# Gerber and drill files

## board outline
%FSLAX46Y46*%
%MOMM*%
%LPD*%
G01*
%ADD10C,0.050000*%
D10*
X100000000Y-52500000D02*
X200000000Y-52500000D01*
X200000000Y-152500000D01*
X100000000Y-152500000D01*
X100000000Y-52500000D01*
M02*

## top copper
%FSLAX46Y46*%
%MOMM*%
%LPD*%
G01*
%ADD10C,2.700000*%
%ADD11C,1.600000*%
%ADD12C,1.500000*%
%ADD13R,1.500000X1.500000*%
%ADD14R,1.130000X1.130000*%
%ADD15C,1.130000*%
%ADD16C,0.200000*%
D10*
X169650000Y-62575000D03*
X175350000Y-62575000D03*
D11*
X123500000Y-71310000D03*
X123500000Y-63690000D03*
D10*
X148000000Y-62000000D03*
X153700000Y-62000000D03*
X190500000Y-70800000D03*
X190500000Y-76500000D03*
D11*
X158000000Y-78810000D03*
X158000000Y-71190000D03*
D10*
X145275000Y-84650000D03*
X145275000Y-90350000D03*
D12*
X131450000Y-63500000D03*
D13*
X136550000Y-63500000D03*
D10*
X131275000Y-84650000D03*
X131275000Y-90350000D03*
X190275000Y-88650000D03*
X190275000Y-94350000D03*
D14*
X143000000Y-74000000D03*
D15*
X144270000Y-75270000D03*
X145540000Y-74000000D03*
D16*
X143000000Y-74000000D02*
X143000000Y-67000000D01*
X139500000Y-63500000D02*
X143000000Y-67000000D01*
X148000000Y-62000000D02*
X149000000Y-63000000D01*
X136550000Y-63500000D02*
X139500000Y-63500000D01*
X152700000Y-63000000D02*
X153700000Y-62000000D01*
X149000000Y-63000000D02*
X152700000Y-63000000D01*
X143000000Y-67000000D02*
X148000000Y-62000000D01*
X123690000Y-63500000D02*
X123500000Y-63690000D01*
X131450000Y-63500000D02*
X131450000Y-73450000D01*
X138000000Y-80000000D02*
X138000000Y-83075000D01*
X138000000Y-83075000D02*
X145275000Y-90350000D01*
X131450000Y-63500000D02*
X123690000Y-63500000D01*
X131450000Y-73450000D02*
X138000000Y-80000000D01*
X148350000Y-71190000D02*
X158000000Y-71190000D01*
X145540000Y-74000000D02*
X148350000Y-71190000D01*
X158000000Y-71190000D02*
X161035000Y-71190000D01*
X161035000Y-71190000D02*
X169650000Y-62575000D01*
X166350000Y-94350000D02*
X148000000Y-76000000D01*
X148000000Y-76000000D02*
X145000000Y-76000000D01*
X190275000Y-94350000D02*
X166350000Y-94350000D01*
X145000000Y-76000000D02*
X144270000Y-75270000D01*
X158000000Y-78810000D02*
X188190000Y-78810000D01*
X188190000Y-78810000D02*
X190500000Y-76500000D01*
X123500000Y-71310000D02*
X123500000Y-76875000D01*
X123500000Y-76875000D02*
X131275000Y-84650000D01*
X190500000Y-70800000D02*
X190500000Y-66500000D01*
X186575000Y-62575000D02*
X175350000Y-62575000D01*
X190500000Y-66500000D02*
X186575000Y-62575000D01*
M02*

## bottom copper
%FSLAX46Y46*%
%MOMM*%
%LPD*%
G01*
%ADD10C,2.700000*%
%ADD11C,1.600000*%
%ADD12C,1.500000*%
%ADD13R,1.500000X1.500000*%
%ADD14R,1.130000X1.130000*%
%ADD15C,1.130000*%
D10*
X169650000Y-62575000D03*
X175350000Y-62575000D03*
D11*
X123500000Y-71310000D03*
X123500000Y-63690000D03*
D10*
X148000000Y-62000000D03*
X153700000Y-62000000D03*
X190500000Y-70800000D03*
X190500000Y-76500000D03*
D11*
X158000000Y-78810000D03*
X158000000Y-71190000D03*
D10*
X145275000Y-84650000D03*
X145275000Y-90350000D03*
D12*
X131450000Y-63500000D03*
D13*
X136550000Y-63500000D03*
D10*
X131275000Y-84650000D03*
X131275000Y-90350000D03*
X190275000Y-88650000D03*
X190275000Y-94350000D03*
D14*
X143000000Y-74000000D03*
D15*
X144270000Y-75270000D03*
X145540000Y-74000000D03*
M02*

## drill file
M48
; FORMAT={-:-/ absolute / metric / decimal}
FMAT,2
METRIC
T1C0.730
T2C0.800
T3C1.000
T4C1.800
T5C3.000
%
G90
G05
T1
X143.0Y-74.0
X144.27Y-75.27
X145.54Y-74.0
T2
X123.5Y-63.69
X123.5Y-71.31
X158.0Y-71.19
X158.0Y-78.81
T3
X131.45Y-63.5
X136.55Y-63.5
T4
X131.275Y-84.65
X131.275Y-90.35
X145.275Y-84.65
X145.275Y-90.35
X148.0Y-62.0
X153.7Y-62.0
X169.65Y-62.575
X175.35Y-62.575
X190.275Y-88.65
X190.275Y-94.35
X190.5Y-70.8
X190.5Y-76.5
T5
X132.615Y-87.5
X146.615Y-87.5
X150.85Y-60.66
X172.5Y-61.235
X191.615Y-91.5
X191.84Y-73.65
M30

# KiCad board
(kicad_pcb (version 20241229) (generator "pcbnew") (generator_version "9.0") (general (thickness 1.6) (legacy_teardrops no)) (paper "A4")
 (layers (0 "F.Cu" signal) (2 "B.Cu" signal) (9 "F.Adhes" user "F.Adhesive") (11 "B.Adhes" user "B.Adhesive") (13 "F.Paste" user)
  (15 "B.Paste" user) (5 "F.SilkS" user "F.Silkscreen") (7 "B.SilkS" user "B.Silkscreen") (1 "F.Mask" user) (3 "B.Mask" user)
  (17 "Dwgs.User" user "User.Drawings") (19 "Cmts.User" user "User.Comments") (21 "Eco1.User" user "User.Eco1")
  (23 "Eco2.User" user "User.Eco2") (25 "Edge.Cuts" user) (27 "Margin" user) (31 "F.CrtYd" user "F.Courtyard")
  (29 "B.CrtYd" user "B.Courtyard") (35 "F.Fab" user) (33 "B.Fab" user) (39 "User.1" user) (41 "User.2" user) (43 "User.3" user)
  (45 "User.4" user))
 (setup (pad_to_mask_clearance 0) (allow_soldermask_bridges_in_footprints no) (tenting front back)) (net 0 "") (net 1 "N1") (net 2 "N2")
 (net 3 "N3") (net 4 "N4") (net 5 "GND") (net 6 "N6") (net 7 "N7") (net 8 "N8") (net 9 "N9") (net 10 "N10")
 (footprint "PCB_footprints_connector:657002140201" (layer "F.Cu") (at 172.5 62.575 180)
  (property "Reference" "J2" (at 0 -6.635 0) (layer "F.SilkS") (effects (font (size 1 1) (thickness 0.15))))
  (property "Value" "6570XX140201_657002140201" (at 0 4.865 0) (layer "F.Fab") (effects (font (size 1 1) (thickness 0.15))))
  (pad "" np_thru_hole circle (at 0 1.34 180) (size 3 3) (drill 3) (layers "*.Cu" "*.Mask"))
  (pad "1" thru_hole circle (at 2.85 0 180) (size 2.7 2.7) (drill 1.8) (layers "*.Cu" "*.Mask") (remove_unused_layers no) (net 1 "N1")
   (solder_mask_margin 0.102))
  (pad "2" thru_hole circle (at -2.85 0 180) (size 2.7 2.7) (drill 1.8) (layers "*.Cu" "*.Mask") (remove_unused_layers no) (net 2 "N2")
   (solder_mask_margin 0.102)))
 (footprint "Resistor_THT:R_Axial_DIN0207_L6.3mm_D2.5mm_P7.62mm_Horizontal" (layer "F.Cu") (at 123.5 71.31 90)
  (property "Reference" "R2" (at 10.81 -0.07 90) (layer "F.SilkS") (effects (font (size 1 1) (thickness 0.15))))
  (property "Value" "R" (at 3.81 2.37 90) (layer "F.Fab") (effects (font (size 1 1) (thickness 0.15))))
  (pad "1" thru_hole circle (at 0 0 90) (size 1.6 1.6) (drill 0.8) (layers "*.Cu" "*.Mask") (remove_unused_layers no) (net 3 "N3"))
  (pad "2" thru_hole circle (at 7.62 0 90) (size 1.6 1.6) (drill 0.8) (layers "*.Cu" "*.Mask") (remove_unused_layers no) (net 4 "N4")))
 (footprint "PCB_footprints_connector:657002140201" (layer "F.Cu") (at 150.85 62 180)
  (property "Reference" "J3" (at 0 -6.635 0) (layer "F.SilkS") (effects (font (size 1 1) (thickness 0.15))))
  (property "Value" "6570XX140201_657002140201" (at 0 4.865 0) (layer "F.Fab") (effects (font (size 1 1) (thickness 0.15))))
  (pad "" np_thru_hole circle (at 0 1.34 180) (size 3 3) (drill 3) (layers "*.Cu" "*.Mask"))
  (pad "1" thru_hole circle (at 2.85 0 180) (size 2.7 2.7) (drill 1.8) (layers "*.Cu" "*.Mask") (remove_unused_layers no) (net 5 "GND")
   (solder_mask_margin 0.102))
  (pad "2" thru_hole circle (at -2.85 0 180) (size 2.7 2.7) (drill 1.8) (layers "*.Cu" "*.Mask") (remove_unused_layers no) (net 5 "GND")
   (solder_mask_margin 0.102)))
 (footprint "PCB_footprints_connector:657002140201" (layer "F.Cu") (at 190.5 73.65 90)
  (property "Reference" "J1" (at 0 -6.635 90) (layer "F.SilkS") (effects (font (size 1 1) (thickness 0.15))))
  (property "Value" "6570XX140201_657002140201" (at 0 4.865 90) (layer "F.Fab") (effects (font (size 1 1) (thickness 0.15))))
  (pad "" np_thru_hole circle (at 0 1.34 90) (size 3 3) (drill 3) (layers "*.Cu" "*.Mask"))
  (pad "1" thru_hole circle (at 2.85 0 90) (size 2.7 2.7) (drill 1.8) (layers "*.Cu" "*.Mask") (remove_unused_layers no) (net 2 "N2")
   (solder_mask_margin 0.102))
  (pad "2" thru_hole circle (at -2.85 0 90) (size 2.7 2.7) (drill 1.8) (layers "*.Cu" "*.Mask") (remove_unused_layers no) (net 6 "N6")
   (solder_mask_margin 0.102)))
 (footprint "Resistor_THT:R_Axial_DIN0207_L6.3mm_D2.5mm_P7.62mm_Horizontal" (layer "F.Cu") (at 158 78.81 90)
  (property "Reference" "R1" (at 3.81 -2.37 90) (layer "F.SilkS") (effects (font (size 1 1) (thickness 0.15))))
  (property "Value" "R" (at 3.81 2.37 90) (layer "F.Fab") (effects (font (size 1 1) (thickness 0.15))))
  (pad "1" thru_hole circle (at 0 0 90) (size 1.6 1.6) (drill 0.8) (layers "*.Cu" "*.Mask") (remove_unused_layers no) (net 6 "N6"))
  (pad "2" thru_hole circle (at 7.62 0 90) (size 1.6 1.6) (drill 0.8) (layers "*.Cu" "*.Mask") (remove_unused_layers no) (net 1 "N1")))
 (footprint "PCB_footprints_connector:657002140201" (layer "F.Cu") (at 145.275 87.5 90)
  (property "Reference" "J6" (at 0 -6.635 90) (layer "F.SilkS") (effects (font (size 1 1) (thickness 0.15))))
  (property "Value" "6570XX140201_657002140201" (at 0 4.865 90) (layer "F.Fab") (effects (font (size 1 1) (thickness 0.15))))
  (pad "" np_thru_hole circle (at 0 1.34 90) (size 3 3) (drill 3) (layers "*.Cu" "*.Mask"))
  (pad "1" thru_hole circle (at 2.85 0 90) (size 2.7 2.7) (drill 1.8) (layers "*.Cu" "*.Mask") (remove_unused_layers no) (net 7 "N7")
   (solder_mask_margin 0.102))
  (pad "2" thru_hole circle (at -2.85 0 90) (size 2.7 2.7) (drill 1.8) (layers "*.Cu" "*.Mask") (remove_unused_layers no) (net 4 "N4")
   (solder_mask_margin 0.102)))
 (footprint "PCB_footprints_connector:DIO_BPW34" (layer "F.Cu") (at 134 63.5 180)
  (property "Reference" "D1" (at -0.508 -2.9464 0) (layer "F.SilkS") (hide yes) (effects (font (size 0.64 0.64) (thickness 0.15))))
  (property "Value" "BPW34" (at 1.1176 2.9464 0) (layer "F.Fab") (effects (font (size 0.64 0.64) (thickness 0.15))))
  (pad "A" thru_hole circle (at 2.55 0 180) (size 1.5 1.5) (drill 1) (layers "*.Cu" "*.Mask") (remove_unused_layers no) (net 4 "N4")
   (solder_mask_margin 0.102))
  (pad "C" thru_hole rect (at -2.55 0 180) (size 1.5 1.5) (drill 1) (layers "*.Cu" "*.Mask") (remove_unused_layers no) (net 5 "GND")
   (solder_mask_margin 0.102)))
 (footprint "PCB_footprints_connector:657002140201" (layer "F.Cu") (at 131.275 87.5 90)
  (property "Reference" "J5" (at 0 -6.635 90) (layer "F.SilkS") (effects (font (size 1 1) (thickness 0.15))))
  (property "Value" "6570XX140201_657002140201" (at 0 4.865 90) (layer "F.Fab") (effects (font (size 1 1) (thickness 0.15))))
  (pad "" np_thru_hole circle (at 0 1.34 90) (size 3 3) (drill 3) (layers "*.Cu" "*.Mask"))
  (pad "1" thru_hole circle (at 2.85 0 90) (size 2.7 2.7) (drill 1.8) (layers "*.Cu" "*.Mask") (remove_unused_layers no) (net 3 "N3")
   (solder_mask_margin 0.102))
  (pad "2" thru_hole circle (at -2.85 0 90) (size 2.7 2.7) (drill 1.8) (layers "*.Cu" "*.Mask") (remove_unused_layers no) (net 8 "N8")
   (solder_mask_margin 0.102)))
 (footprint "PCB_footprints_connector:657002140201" (layer "F.Cu") (at 190.275 91.5 90)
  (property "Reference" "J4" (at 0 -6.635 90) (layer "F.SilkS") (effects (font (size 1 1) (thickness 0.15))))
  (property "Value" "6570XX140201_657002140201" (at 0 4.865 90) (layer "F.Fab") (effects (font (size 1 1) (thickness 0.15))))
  (pad "" np_thru_hole circle (at 0 1.34 90) (size 3 3) (drill 3) (layers "*.Cu" "*.Mask"))
  (pad "1" thru_hole circle (at 2.85 0 90) (size 2.7 2.7) (drill 1.8) (layers "*.Cu" "*.Mask") (remove_unused_layers no) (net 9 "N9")
   (solder_mask_margin 0.102))
  (pad "2" thru_hole circle (at -2.85 0 90) (size 2.7 2.7) (drill 1.8) (layers "*.Cu" "*.Mask") (remove_unused_layers no) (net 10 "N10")
   (solder_mask_margin 0.102)))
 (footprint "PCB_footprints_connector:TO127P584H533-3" (layer "F.Cu") (at 144.27 74)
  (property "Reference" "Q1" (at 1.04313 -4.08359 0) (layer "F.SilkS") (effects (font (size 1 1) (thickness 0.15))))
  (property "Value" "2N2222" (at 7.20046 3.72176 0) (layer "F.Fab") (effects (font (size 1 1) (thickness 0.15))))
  (pad "1" thru_hole rect (at -1.27 0) (size 1.13 1.13) (drill 0.73) (layers "*.Cu" "*.Mask") (remove_unused_layers no) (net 5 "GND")
   (solder_mask_margin 0.102))
  (pad "2" thru_hole circle (at 0 1.27) (size 1.13 1.13) (drill 0.73) (layers "*.Cu" "*.Mask") (remove_unused_layers no) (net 10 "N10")
   (solder_mask_margin 0.102))
  (pad "3" thru_hole circle (at 1.27 0) (size 1.13 1.13) (drill 0.73) (layers "*.Cu" "*.Mask") (remove_unused_layers no) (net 1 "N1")
   (solder_mask_margin 0.102)))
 (gr_rect (start 100 52.5) (end 200 152.5) (stroke (width 0.05) (type default)) (fill no) (layer "Edge.Cuts"))
 (segment (start 143 74) (end 143 67) (width 0.2) (layer "F.Cu") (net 5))
 (segment (start 139.5 63.5) (end 143 67) (width 0.2) (layer "F.Cu") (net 5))
 (segment (start 148 62) (end 149 63) (width 0.2) (layer "F.Cu") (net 5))
 (segment (start 136.55 63.5) (end 139.5 63.5) (width 0.2) (layer "F.Cu") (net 5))
 (segment (start 152.7 63) (end 153.7 62) (width 0.2) (layer "F.Cu") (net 5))
 (segment (start 149 63) (end 152.7 63) (width 0.2) (layer "F.Cu") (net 5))
 (segment (start 143 67) (end 148 62) (width 0.2) (layer "F.Cu") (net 5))
 (segment (start 123.69 63.5) (end 123.5 63.69) (width 0.2) (layer "F.Cu") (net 4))
 (segment (start 131.45 63.5) (end 131.45 73.45) (width 0.2) (layer "F.Cu") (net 4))
 (segment (start 138 80) (end 138 83.075) (width 0.2) (layer "F.Cu") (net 4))
 (segment (start 138 83.075) (end 145.275 90.35) (width 0.2) (layer "F.Cu") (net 4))
 (segment (start 131.45 63.5) (end 123.69 63.5) (width 0.2) (layer "F.Cu") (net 4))
 (segment (start 131.45 73.45) (end 138 80) (width 0.2) (layer "F.Cu") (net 4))
 (segment (start 148.35 71.19) (end 158 71.19) (width 0.2) (layer "F.Cu") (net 1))
 (segment (start 145.54 74) (end 148.35 71.19) (width 0.2) (layer "F.Cu") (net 1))
 (segment (start 158 71.19) (end 161.035 71.19) (width 0.2) (layer "F.Cu") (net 1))
 (segment (start 161.035 71.19) (end 169.65 62.575) (width 0.2) (layer "F.Cu") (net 1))
 (segment (start 166.35 94.35) (end 148 76) (width 0.2) (layer "F.Cu") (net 10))
 (segment (start 148 76) (end 145 76) (width 0.2) (layer "F.Cu") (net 10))
 (segment (start 190.275 94.35) (end 166.35 94.35) (width 0.2) (layer "F.Cu") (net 10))
 (segment (start 145 76) (end 144.27 75.27) (width 0.2) (layer "F.Cu") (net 10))
 (segment (start 158 78.81) (end 188.19 78.81) (width 0.2) (layer "F.Cu") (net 6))
 (segment (start 188.19 78.81) (end 190.5 76.5) (width 0.2) (layer "F.Cu") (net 6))
 (segment (start 123.5 71.31) (end 123.5 76.875) (width 0.2) (layer "F.Cu") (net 3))
 (segment (start 123.5 76.875) (end 131.275 84.65) (width 0.2) (layer "F.Cu") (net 3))
 (segment (start 190.5 70.8) (end 190.5 66.5) (width 0.2) (layer "F.Cu") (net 2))
 (segment (start 186.575 62.575) (end 175.35 62.575) (width 0.2) (layer "F.Cu") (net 2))
 (segment (start 190.5 66.5) (end 186.575 62.575) (width 0.2) (layer "F.Cu") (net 2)))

